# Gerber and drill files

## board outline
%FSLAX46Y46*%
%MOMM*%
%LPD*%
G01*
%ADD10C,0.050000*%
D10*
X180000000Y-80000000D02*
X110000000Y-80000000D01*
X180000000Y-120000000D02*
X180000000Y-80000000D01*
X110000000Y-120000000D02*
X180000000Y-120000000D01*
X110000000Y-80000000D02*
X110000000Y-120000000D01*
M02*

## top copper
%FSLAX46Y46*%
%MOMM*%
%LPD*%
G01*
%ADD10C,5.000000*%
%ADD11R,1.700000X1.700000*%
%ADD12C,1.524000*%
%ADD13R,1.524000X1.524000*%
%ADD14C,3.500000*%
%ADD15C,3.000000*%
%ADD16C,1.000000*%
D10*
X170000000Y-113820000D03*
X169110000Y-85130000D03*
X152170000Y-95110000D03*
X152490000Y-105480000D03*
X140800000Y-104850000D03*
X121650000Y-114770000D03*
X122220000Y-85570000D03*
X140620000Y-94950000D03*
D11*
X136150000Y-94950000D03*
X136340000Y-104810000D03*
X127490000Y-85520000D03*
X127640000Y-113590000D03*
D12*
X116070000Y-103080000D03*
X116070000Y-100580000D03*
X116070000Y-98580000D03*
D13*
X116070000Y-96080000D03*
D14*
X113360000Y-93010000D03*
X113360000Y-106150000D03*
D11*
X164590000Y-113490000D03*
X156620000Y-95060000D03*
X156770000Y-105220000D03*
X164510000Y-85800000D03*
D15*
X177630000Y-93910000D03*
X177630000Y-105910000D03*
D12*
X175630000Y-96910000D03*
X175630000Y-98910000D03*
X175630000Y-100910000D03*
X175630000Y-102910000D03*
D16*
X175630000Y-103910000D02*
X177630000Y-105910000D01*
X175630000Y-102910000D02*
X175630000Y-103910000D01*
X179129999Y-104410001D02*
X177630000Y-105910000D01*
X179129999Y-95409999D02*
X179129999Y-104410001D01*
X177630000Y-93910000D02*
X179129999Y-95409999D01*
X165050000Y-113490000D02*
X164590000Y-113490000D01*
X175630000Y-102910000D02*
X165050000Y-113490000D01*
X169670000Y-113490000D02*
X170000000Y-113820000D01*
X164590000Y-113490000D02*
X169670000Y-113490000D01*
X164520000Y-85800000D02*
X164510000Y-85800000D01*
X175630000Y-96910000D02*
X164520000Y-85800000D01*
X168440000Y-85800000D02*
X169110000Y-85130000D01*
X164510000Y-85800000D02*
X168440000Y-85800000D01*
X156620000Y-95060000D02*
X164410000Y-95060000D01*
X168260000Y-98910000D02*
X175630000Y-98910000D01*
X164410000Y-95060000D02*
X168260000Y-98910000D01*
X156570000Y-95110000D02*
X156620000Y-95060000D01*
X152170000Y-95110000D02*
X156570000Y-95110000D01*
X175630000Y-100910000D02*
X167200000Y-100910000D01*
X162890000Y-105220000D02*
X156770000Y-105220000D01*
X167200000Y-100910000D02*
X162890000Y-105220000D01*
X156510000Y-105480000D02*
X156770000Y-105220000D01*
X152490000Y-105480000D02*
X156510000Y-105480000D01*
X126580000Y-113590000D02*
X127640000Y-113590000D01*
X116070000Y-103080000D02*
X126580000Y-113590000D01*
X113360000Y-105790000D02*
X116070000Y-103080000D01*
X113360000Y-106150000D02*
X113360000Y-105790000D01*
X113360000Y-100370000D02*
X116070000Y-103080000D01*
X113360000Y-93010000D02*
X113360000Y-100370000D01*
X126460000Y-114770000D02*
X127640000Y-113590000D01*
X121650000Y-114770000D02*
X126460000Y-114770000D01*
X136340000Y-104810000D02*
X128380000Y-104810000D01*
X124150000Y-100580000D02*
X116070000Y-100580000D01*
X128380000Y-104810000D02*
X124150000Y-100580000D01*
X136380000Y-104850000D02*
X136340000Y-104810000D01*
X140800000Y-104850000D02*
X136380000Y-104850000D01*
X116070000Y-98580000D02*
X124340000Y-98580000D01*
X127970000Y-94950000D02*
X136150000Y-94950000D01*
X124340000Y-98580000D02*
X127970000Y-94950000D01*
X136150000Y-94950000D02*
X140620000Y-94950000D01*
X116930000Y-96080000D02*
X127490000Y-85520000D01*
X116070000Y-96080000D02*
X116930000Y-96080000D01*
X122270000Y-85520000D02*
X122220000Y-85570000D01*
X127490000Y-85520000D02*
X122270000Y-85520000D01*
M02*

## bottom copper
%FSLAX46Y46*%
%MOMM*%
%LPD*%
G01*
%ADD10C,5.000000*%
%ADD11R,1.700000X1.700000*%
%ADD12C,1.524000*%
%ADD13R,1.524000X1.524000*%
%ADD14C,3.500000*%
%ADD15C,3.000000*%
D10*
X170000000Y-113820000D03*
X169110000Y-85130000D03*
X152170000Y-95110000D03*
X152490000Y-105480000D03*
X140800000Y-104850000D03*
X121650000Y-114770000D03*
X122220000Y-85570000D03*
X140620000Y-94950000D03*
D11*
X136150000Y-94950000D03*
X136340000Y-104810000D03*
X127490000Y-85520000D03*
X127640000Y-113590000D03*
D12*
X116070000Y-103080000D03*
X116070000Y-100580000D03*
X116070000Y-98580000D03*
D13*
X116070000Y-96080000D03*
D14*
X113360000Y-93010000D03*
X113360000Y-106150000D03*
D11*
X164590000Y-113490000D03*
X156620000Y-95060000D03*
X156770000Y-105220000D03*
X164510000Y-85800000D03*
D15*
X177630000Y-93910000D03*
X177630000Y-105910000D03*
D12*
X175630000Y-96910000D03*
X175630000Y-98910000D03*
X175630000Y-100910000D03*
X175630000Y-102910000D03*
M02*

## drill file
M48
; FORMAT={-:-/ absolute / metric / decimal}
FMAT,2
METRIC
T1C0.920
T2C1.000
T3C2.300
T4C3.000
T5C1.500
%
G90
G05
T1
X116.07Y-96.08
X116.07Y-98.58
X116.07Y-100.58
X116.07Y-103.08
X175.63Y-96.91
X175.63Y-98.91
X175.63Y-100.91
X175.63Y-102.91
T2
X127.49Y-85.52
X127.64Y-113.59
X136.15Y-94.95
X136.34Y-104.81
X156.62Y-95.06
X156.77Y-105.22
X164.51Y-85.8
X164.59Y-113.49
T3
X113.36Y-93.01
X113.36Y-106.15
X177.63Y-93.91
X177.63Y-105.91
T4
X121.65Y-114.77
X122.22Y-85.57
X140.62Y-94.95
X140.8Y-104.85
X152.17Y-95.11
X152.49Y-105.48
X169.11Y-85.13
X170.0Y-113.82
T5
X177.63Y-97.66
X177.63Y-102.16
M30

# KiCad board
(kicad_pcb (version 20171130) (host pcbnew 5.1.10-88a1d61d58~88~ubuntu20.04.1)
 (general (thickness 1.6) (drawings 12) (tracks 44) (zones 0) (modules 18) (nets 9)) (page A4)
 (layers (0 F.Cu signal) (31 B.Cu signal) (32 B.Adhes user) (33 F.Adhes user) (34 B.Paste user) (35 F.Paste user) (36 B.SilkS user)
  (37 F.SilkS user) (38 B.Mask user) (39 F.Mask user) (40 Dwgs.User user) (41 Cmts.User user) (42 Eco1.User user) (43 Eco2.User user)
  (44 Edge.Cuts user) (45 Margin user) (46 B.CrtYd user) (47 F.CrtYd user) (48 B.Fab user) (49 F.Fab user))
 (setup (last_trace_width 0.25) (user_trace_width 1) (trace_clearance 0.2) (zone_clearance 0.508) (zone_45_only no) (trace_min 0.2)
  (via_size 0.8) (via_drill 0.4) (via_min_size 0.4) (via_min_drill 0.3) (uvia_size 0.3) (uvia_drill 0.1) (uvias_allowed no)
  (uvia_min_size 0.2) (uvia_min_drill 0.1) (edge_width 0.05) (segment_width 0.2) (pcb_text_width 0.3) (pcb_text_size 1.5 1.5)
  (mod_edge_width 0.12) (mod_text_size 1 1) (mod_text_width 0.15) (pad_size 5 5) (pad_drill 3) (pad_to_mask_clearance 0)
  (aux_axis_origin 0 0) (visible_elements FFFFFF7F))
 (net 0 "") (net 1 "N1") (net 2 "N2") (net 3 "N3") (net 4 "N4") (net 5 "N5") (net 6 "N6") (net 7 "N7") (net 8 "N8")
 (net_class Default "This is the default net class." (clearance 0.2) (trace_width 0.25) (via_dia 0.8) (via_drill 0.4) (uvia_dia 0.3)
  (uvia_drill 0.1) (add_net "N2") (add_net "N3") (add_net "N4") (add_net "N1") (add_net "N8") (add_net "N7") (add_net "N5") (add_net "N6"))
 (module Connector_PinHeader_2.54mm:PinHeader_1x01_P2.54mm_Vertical (layer F.Cu) (at 170 113.82 90)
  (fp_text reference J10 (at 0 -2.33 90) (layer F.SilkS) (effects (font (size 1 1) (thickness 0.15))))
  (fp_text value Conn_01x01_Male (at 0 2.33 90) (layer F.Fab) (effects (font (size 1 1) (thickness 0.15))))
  (pad 1 thru_hole circle (at 0 0 90) (size 5 5) (drill 3) (layers *.Cu *.Mask) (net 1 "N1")))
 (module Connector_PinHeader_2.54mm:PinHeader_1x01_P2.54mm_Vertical (layer F.Cu) (at 169.11 85.13 90)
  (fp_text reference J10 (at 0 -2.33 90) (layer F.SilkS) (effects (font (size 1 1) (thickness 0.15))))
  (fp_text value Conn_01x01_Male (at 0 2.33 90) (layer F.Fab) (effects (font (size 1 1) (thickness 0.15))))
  (pad 1 thru_hole circle (at 0 0 90) (size 5 5) (drill 3) (layers *.Cu *.Mask) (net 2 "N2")))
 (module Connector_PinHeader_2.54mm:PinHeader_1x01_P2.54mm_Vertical (layer F.Cu) (at 152.17 95.11 90)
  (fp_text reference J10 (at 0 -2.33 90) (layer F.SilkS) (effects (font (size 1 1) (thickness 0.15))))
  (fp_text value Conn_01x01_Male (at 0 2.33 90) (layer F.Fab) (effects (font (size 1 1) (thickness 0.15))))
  (pad 1 thru_hole circle (at 0 0 90) (size 5 5) (drill 3) (layers *.Cu *.Mask) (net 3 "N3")))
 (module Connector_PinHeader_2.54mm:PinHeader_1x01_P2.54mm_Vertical (layer F.Cu) (at 152.49 105.48 90)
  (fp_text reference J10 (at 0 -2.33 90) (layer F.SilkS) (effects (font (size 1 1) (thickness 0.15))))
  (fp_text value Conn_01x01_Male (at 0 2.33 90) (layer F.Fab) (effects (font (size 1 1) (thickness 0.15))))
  (pad 1 thru_hole circle (at 0 0 90) (size 5 5) (drill 3) (layers *.Cu *.Mask) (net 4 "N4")))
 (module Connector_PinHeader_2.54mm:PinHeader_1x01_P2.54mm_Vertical (layer F.Cu) (at 140.8 104.85 90)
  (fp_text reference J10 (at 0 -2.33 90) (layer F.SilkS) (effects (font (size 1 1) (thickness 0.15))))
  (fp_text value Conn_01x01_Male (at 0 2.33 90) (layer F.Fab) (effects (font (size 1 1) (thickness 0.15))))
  (pad 1 thru_hole circle (at 0 0 90) (size 5 5) (drill 3) (layers *.Cu *.Mask) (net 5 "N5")))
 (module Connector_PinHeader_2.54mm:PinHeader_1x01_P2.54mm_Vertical (layer F.Cu) (at 121.65 114.77 90)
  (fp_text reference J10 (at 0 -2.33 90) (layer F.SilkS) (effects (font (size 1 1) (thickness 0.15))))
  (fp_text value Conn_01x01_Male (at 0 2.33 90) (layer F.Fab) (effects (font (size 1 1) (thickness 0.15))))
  (pad 1 thru_hole circle (at 0 0 90) (size 5 5) (drill 3) (layers *.Cu *.Mask) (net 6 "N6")))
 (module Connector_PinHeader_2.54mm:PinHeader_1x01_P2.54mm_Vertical (layer F.Cu) (at 122.22 85.57 90)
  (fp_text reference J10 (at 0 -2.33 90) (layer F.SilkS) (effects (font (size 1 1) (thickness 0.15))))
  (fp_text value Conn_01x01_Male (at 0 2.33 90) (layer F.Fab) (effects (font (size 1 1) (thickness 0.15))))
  (pad 1 thru_hole circle (at 0 0 90) (size 5 5) (drill 3) (layers *.Cu *.Mask) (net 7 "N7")))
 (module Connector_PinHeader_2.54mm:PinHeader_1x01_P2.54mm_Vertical (layer F.Cu) (at 140.62 94.95 90)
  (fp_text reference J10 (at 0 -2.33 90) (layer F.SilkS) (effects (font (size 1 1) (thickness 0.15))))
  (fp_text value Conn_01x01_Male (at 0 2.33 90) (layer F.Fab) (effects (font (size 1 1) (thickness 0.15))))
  (pad 1 thru_hole circle (at 0 0 90) (size 5 5) (drill 3) (layers *.Cu *.Mask) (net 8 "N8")))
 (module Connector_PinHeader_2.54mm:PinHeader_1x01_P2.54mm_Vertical (layer F.Cu) (at 136.15 94.95 90)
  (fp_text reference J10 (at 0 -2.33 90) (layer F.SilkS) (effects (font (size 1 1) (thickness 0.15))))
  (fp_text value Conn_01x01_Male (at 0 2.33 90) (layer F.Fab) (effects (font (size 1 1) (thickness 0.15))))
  (pad 1 thru_hole rect (at 0 0 90) (size 1.7 1.7) (drill 1) (layers *.Cu *.Mask) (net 8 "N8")))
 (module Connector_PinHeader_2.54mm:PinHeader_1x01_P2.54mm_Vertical (layer F.Cu) (at 136.34 104.81 90)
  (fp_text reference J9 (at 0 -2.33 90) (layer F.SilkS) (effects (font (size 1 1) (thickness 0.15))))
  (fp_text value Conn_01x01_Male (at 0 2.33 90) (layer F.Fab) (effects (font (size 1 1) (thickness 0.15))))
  (pad 1 thru_hole rect (at 0 0 90) (size 1.7 1.7) (drill 1) (layers *.Cu *.Mask) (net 5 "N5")))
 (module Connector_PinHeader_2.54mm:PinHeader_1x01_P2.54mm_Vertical (layer F.Cu) (at 127.49 85.52 90)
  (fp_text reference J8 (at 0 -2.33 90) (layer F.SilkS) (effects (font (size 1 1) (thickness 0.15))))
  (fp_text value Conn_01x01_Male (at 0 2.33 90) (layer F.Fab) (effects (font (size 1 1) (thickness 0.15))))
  (pad 1 thru_hole rect (at 0 0 90) (size 1.7 1.7) (drill 1) (layers *.Cu *.Mask) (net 7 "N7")))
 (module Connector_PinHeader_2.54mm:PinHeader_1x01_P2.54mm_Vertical (layer F.Cu) (at 127.64 113.59 90)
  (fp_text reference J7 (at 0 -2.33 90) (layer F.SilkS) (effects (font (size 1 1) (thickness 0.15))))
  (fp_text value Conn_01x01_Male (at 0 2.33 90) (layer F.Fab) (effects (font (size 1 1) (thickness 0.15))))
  (pad 1 thru_hole rect (at 0 0 90) (size 1.7 1.7) (drill 1) (layers *.Cu *.Mask) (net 6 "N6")))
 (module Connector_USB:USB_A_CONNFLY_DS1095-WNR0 (layer F.Cu) (at 116.07 96.08 270)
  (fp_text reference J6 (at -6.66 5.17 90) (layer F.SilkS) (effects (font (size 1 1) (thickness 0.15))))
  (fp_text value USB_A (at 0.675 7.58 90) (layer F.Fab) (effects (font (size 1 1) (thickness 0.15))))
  (pad 4 thru_hole circle (at 7 0 270) (size 1.524 1.524) (drill 0.92) (layers *.Cu *.Mask) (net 6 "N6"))
  (pad 3 thru_hole circle (at 4.5 0 270) (size 1.524 1.524) (drill 0.92) (layers *.Cu *.Mask) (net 5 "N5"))
  (pad 2 thru_hole circle (at 2.5 0 270) (size 1.524 1.524) (drill 0.92) (layers *.Cu *.Mask) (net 8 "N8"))
  (pad 1 thru_hole rect (at 0 0 270) (size 1.524 1.524) (drill 0.92) (layers *.Cu *.Mask) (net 7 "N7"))
  (pad 5 thru_hole circle (at -3.07 2.71 270) (size 3.5 3.5) (drill 2.3) (layers *.Cu *.Mask) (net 6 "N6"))
  (pad 5 thru_hole circle (at 10.07 2.71 270) (size 3.5 3.5) (drill 2.3) (layers *.Cu *.Mask) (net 6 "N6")))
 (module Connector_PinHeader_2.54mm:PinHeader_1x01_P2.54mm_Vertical (layer F.Cu) (at 164.59 113.49 90)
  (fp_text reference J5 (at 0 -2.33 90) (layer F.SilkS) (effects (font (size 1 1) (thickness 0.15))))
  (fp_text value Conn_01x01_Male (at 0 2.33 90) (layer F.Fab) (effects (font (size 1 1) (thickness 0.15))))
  (pad 1 thru_hole rect (at 0 0 90) (size 1.7 1.7) (drill 1) (layers *.Cu *.Mask) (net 1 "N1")))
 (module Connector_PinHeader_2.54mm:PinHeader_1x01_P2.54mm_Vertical (layer F.Cu) (at 156.62 95.06 90)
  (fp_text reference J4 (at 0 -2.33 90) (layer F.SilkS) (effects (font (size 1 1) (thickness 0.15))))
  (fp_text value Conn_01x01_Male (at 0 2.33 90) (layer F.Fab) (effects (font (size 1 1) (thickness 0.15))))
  (pad 1 thru_hole rect (at 0 0 90) (size 1.7 1.7) (drill 1) (layers *.Cu *.Mask) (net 3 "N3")))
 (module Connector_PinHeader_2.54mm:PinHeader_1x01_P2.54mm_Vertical (layer F.Cu) (at 156.77 105.22 90)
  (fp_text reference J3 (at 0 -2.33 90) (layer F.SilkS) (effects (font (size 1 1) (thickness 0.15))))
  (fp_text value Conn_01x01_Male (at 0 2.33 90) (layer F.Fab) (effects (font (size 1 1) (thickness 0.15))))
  (pad 1 thru_hole rect (at 0 0 90) (size 1.7 1.7) (drill 1) (layers *.Cu *.Mask) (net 4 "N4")))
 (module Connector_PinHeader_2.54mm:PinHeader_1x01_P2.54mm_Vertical (layer F.Cu) (at 164.51 85.8 90)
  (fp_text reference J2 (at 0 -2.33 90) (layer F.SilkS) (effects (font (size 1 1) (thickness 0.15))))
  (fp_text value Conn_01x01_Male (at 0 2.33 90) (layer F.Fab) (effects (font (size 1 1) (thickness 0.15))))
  (pad 1 thru_hole rect (at 0 0 90) (size 1.7 1.7) (drill 1) (layers *.Cu *.Mask) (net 2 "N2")))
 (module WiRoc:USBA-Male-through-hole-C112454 (layer F.Cu) (at 177.63 99.91 90)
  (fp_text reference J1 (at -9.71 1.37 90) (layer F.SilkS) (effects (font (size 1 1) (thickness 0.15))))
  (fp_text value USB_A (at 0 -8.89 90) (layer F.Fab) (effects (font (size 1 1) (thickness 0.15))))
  (pad "" np_thru_hole circle (at 2.25 0 90) (size 1.5 1.5) (drill 1.5) (layers *.Cu *.Mask))
  (pad "" np_thru_hole circle (at -2.25 0 90) (size 1.5 1.5) (drill 1.5) (layers *.Cu *.Mask))
  (pad 5 thru_hole circle (at 6 0 90) (size 3 3) (drill 2.3) (layers *.Cu *.Mask) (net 1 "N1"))
  (pad 5 thru_hole circle (at -6 0 90) (size 3 3) (drill 2.3) (layers *.Cu *.Mask) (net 1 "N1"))
  (pad 1 thru_hole circle (at 3 -2 90) (size 1.524 1.524) (drill 0.92) (layers *.Cu *.Mask) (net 2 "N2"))
  (pad 2 thru_hole circle (at 1 -2 90) (size 1.524 1.524) (drill 0.92) (layers *.Cu *.Mask) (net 3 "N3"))
  (pad 3 thru_hole circle (at -1 -2 90) (size 1.524 1.524) (drill 0.92) (layers *.Cu *.Mask) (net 4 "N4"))
  (pad 4 thru_hole circle (at -3 -2 90) (size 1.524 1.524) (drill 0.92) (layers *.Cu *.Mask) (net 1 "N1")))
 (gr_line (start 180 80) (end 110 80) (layer Edge.Cuts) (width 0.05))
 (gr_line (start 180 120) (end 180 80) (layer Edge.Cuts) (width 0.05))
 (gr_line (start 110 120) (end 180 120) (layer Edge.Cuts) (width 0.05))
 (gr_line (start 110 80) (end 110 120) (layer Edge.Cuts) (width 0.05))
 (segment (start 175.63 103.91) (end 177.63 105.91) (width 1) (layer F.Cu) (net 1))
 (segment (start 175.63 102.91) (end 175.63 103.91) (width 1) (layer F.Cu) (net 1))
 (segment (start 179.129999 104.410001) (end 177.63 105.91) (width 1) (layer F.Cu) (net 1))
 (segment (start 179.129999 95.409999) (end 179.129999 104.410001) (width 1) (layer F.Cu) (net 1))
 (segment (start 177.63 93.91) (end 179.129999 95.409999) (width 1) (layer F.Cu) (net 1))
 (segment (start 165.05 113.49) (end 164.59 113.49) (width 1) (layer F.Cu) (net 1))
 (segment (start 175.63 102.91) (end 165.05 113.49) (width 1) (layer F.Cu) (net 1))
 (segment (start 169.67 113.49) (end 170 113.82) (width 1) (layer F.Cu) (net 1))
 (segment (start 164.59 113.49) (end 169.67 113.49) (width 1) (layer F.Cu) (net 1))
 (segment (start 164.52 85.8) (end 164.51 85.8) (width 1) (layer F.Cu) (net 2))
 (segment (start 175.63 96.91) (end 164.52 85.8) (width 1) (layer F.Cu) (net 2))
 (segment (start 168.44 85.8) (end 169.11 85.13) (width 1) (layer F.Cu) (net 2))
 (segment (start 164.51 85.8) (end 168.44 85.8) (width 1) (layer F.Cu) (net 2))
 (segment (start 156.62 95.06) (end 164.41 95.06) (width 1) (layer F.Cu) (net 3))
 (segment (start 168.26 98.91) (end 175.63 98.91) (width 1) (layer F.Cu) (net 3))
 (segment (start 164.41 95.06) (end 168.26 98.91) (width 1) (layer F.Cu) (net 3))
 (segment (start 156.57 95.11) (end 156.62 95.06) (width 1) (layer F.Cu) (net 3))
 (segment (start 152.17 95.11) (end 156.57 95.11) (width 1) (layer F.Cu) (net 3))
 (segment (start 175.63 100.91) (end 167.2 100.91) (width 1) (layer F.Cu) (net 4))
 (segment (start 162.89 105.22) (end 156.77 105.22) (width 1) (layer F.Cu) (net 4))
 (segment (start 167.2 100.91) (end 162.89 105.22) (width 1) (layer F.Cu) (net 4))
 (segment (start 156.51 105.48) (end 156.77 105.22) (width 1) (layer F.Cu) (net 4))
 (segment (start 152.49 105.48) (end 156.51 105.48) (width 1) (layer F.Cu) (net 4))
 (segment (start 126.58 113.59) (end 127.64 113.59) (width 1) (layer F.Cu) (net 6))
 (segment (start 116.07 103.08) (end 126.58 113.59) (width 1) (layer F.Cu) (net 6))
 (segment (start 113.36 105.79) (end 116.07 103.08) (width 1) (layer F.Cu) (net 6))
 (segment (start 113.36 106.15) (end 113.36 105.79) (width 1) (layer F.Cu) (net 6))
 (segment (start 113.36 100.37) (end 116.07 103.08) (width 1) (layer F.Cu) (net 6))
 (segment (start 113.36 93.01) (end 113.36 100.37) (width 1) (layer F.Cu) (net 6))
 (segment (start 126.46 114.77) (end 127.64 113.59) (width 1) (layer F.Cu) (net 6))
 (segment (start 121.65 114.77) (end 126.46 114.77) (width 1) (layer F.Cu) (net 6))
 (segment (start 136.34 104.81) (end 128.38 104.81) (width 1) (layer F.Cu) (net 5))
 (segment (start 124.15 100.58) (end 116.07 100.58) (width 1) (layer F.Cu) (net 5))
 (segment (start 128.38 104.81) (end 124.15 100.58) (width 1) (layer F.Cu) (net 5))
 (segment (start 136.38 104.85) (end 136.34 104.81) (width 1) (layer F.Cu) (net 5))
 (segment (start 140.8 104.85) (end 136.38 104.85) (width 1) (layer F.Cu) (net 5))
 (segment (start 116.07 98.58) (end 124.34 98.58) (width 1) (layer F.Cu) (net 8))
 (segment (start 127.97 94.95) (end 136.15 94.95) (width 1) (layer F.Cu) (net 8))
 (segment (start 124.34 98.58) (end 127.97 94.95) (width 1) (layer F.Cu) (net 8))
 (segment (start 136.15 94.95) (end 140.62 94.95) (width 1) (layer F.Cu) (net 8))
 (segment (start 116.93 96.08) (end 127.49 85.52) (width 1) (layer F.Cu) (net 7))
 (segment (start 116.07 96.08) (end 116.93 96.08) (width 1) (layer F.Cu) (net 7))
 (segment (start 122.27 85.52) (end 122.22 85.57) (width 1) (layer F.Cu) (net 7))
 (segment (start 127.49 85.52) (end 122.27 85.52) (width 1) (layer F.Cu) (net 7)))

